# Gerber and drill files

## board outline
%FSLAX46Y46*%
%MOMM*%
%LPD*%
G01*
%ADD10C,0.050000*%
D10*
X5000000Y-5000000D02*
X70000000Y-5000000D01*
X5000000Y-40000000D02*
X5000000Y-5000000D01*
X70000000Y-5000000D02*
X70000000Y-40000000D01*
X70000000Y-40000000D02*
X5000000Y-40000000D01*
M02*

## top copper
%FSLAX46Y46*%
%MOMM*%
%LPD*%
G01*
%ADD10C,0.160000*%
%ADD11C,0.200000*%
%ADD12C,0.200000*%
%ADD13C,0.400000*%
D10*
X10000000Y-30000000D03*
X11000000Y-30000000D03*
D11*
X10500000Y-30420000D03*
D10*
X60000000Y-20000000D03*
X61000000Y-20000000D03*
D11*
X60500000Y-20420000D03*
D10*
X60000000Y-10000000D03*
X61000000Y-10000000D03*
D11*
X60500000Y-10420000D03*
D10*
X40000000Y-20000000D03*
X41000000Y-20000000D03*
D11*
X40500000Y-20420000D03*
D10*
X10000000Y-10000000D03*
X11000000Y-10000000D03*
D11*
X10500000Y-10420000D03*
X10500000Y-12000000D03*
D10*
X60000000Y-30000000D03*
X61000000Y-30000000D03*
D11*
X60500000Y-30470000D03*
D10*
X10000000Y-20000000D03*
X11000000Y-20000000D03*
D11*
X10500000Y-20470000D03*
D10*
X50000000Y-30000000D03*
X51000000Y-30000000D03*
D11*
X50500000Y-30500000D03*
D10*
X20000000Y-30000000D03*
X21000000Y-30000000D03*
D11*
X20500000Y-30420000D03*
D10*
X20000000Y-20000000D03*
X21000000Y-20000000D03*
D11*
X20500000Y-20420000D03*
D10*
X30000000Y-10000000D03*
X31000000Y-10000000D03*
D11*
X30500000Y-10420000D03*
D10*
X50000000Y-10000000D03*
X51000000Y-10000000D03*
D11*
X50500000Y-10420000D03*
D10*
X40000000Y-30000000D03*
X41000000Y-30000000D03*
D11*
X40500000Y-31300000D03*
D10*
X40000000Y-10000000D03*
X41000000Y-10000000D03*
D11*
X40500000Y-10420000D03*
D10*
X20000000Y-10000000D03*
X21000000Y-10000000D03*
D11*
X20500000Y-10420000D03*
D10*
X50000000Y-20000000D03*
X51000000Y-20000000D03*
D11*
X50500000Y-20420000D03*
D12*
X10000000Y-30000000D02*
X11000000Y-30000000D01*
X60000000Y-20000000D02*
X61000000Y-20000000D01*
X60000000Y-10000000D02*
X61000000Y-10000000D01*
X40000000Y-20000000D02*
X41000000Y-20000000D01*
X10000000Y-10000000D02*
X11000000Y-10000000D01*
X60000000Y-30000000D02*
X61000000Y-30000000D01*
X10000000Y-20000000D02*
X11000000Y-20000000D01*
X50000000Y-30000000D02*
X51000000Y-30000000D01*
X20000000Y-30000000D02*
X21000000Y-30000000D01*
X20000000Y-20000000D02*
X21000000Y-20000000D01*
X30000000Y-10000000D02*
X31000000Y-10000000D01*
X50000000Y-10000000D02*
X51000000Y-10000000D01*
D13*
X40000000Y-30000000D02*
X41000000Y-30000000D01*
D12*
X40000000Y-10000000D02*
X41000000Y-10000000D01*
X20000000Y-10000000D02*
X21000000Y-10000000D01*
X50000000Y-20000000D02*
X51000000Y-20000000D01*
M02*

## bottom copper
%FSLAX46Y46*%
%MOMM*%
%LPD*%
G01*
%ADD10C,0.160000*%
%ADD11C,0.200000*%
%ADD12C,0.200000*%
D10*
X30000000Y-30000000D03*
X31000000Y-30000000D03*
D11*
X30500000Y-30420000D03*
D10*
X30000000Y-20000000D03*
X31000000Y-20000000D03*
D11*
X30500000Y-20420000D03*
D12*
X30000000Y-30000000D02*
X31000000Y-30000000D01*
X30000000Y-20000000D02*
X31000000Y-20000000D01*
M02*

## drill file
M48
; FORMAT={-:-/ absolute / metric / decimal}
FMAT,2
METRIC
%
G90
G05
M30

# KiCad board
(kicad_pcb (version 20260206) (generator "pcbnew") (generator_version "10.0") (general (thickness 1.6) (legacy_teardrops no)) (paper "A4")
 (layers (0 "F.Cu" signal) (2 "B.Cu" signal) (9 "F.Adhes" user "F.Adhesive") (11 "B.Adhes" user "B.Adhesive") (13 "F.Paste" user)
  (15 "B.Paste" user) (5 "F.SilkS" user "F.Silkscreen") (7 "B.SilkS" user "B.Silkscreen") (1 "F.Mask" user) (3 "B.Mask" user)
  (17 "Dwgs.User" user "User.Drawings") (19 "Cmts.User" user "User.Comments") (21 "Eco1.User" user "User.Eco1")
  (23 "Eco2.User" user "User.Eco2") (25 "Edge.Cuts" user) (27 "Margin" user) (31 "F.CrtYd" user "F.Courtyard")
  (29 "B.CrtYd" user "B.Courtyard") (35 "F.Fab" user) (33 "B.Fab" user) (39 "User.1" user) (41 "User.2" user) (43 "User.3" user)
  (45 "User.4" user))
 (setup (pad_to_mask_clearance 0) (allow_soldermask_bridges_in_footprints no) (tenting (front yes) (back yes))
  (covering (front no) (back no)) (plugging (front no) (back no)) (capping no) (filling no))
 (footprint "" (layer "F.Cu") (at 10 30)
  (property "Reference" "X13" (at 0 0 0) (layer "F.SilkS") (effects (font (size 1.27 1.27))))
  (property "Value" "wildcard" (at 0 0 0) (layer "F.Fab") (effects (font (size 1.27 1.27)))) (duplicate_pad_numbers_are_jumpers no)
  (pad "1" smd circle (at 0 0) (size 0.16 0.16) (layers "F.Cu") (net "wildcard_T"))
  (pad "2" smd circle (at 1 0) (size 0.16 0.16) (layers "F.Cu") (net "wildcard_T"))
  (pad "3" smd circle (at 0.5 0.42) (size 0.2 0.2) (layers "F.Cu") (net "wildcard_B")))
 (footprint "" (layer "F.Cu") (at 60 20)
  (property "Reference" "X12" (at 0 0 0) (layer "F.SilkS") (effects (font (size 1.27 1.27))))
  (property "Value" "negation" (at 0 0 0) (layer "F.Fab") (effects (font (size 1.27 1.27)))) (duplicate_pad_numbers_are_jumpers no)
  (pad "1" smd circle (at 0 0) (size 0.16 0.16) (layers "F.Cu") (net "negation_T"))
  (pad "2" smd circle (at 1 0) (size 0.16 0.16) (layers "F.Cu") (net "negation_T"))
  (pad "3" smd circle (at 0.5 0.42) (size 0.2 0.2) (layers "F.Cu") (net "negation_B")))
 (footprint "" (layer "F.Cu") (at 60 10)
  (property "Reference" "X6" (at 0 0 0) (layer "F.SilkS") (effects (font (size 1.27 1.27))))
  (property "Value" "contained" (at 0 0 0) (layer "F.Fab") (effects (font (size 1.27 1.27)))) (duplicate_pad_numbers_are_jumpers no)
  (pad "1" smd circle (at 0 0) (size 0.16 0.16) (layers "F.Cu") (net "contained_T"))
  (pad "2" smd circle (at 1 0) (size 0.16 0.16) (layers "F.Cu") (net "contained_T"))
  (pad "3" smd circle (at 0.5 0.42) (size 0.2 0.2) (layers "F.Cu") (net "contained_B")))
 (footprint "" (layer "F.Cu") (at 40 20)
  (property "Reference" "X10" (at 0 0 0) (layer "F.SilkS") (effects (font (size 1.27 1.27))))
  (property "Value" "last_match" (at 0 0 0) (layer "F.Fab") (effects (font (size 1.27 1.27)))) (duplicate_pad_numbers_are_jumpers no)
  (pad "1" smd circle (at 0 0) (size 0.16 0.16) (layers "F.Cu") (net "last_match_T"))
  (pad "2" smd circle (at 1 0) (size 0.16 0.16) (layers "F.Cu") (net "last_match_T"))
  (pad "3" smd circle (at 0.5 0.42) (size 0.2 0.2) (layers "F.Cu") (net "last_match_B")))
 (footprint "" (layer "F.Cu") (at 10 10)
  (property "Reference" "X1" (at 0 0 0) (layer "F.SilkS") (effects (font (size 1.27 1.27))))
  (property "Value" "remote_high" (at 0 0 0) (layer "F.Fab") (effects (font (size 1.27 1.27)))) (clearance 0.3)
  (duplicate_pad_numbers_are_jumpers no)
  (pad "1" smd circle (at 0 0) (size 0.16 0.16) (layers "F.Cu") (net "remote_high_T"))
  (pad "2" smd circle (at 1 0) (size 0.16 0.16) (layers "F.Cu") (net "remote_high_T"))
  (pad "3" smd circle (at 0.5 0.42) (size 0.2 0.2) (layers "F.Cu") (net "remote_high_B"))
  (pad "4" smd circle (at 0.5 2) (size 0.2 0.2) (layers "F.Cu") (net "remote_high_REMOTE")))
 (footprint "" (layer "F.Cu") (at 60 30)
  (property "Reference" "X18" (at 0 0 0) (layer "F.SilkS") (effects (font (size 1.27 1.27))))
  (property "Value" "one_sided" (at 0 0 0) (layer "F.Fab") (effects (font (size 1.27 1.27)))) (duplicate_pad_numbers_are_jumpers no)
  (pad "1" smd circle (at 0 0) (size 0.16 0.16) (layers "F.Cu") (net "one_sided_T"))
  (pad "2" smd circle (at 1 0) (size 0.16 0.16) (layers "F.Cu") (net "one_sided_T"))
  (pad "3" smd circle (at 0.5 0.47) (size 0.2 0.2) (layers "F.Cu") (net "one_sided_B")))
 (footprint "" (layer "F.Cu") (at 10 20)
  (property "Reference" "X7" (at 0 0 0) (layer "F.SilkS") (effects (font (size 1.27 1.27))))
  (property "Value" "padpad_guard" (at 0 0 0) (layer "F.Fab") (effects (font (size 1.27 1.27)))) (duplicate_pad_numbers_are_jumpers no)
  (pad "1" smd circle (at 0 0) (size 0.16 0.16) (layers "F.Cu") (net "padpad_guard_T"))
  (pad "2" smd circle (at 1 0) (size 0.16 0.16) (layers "F.Cu") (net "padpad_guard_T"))
  (pad "3" smd circle (at 0.5 0.47) (size 0.2 0.2) (layers "F.Cu") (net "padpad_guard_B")))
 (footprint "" (layer "F.Cu") (at 50 30)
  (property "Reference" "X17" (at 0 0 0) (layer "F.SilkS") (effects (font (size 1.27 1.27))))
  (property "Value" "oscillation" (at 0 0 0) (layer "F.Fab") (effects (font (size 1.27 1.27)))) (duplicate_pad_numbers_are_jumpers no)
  (pad "1" smd circle (at 0 0) (size 0.16 0.16) (layers "F.Cu") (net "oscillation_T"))
  (pad "2" smd circle (at 1 0) (size 0.16 0.16) (layers "F.Cu") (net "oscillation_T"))
  (pad "3" smd circle (at 0.5 0.5) (size 0.2 0.2) (layers "F.Cu") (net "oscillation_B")))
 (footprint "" (layer "F.Cu") (at 20 30)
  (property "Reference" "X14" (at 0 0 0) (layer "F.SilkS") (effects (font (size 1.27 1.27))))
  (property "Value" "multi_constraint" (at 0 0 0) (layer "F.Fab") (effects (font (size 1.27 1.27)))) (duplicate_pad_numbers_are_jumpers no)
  (pad "1" smd circle (at 0 0) (size 0.16 0.16) (layers "F.Cu") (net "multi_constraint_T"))
  (pad "2" smd circle (at 1 0) (size 0.16 0.16) (layers "F.Cu") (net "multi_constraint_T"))
  (pad "3" smd circle (at 0.5 0.42) (size 0.2 0.2) (layers "F.Cu") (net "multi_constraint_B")))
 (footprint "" (layer "F.Cu") (at 30 30)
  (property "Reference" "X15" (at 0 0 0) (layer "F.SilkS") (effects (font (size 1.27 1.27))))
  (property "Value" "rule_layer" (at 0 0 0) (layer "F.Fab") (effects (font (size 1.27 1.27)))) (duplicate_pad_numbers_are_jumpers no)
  (pad "1" smd circle (at 0 0) (size 0.16 0.16) (layers "B.Cu") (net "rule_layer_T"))
  (pad "2" smd circle (at 1 0) (size 0.16 0.16) (layers "B.Cu") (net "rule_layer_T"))
  (pad "3" smd circle (at 0.5 0.42) (size 0.2 0.2) (layers "B.Cu") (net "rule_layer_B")))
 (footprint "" (layer "F.Cu") (at 20 20)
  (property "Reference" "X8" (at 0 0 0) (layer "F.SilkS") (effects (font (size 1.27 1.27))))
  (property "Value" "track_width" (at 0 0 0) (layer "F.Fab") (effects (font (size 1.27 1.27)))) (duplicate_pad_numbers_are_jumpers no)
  (pad "1" smd circle (at 0 0) (size 0.16 0.16) (layers "F.Cu") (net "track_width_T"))
  (pad "2" smd circle (at 1 0) (size 0.16 0.16) (layers "F.Cu") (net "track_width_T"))
  (pad "3" smd circle (at 0.5 0.42) (size 0.2 0.2) (layers "F.Cu") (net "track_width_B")))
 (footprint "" (layer "F.Cu") (at 30 10)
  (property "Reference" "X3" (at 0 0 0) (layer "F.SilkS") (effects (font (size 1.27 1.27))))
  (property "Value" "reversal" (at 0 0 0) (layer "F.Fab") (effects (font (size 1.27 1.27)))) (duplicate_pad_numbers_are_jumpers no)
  (pad "1" smd circle (at 0 0) (size 0.16 0.16) (layers "F.Cu") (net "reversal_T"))
  (pad "2" smd circle (at 1 0) (size 0.16 0.16) (layers "F.Cu") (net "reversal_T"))
  (pad "3" smd circle (at 0.5 0.42) (size 0.2 0.2) (layers "F.Cu") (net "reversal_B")))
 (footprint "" (layer "F.Cu") (at 50 10)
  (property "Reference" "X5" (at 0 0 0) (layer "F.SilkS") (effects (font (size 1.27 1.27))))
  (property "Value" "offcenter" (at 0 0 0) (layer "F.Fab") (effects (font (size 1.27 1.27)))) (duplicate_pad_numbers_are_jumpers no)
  (pad "1" smd circle (at 0 0) (size 0.16 0.16) (layers "F.Cu") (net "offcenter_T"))
  (pad "2" smd circle (at 1 0) (size 0.16 0.16) (layers "F.Cu") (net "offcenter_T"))
  (pad "3" smd circle (at 0.5 0.42) (size 0.2 0.2) (layers "F.Cu") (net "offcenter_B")))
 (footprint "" (layer "F.Cu") (at 40 30)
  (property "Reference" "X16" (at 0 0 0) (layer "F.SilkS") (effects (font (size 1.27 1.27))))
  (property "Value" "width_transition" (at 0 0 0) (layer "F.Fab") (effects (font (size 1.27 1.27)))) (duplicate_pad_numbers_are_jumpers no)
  (pad "1" smd circle (at 0 0) (size 0.16 0.16) (layers "F.Cu") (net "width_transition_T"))
  (pad "2" smd circle (at 1 0) (size 0.16 0.16) (layers "F.Cu") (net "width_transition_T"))
  (pad "3" smd circle (at 0.5 1.3) (size 0.2 0.2) (layers "F.Cu") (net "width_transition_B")))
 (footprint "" (layer "F.Cu") (at 30 20)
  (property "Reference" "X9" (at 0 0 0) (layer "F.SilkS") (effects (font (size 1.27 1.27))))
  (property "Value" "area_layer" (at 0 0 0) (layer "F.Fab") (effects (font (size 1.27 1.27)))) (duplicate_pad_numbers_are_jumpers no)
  (pad "1" smd circle (at 0 0) (size 0.16 0.16) (layers "B.Cu") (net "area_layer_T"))
  (pad "2" smd circle (at 1 0) (size 0.16 0.16) (layers "B.Cu") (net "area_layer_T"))
  (pad "3" smd circle (at 0.5 0.42) (size 0.2 0.2) (layers "B.Cu") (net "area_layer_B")))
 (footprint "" (layer "F.Cu") (at 40 10)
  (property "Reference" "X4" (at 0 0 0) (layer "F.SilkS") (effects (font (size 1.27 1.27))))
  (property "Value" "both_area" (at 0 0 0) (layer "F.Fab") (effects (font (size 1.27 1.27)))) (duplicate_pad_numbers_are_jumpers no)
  (pad "1" smd circle (at 0 0) (size 0.16 0.16) (layers "F.Cu") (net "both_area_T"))
  (pad "2" smd circle (at 1 0) (size 0.16 0.16) (layers "F.Cu") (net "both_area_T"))
  (pad "3" smd circle (at 0.5 0.42) (size 0.2 0.2) (layers "F.Cu") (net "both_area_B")))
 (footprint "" (layer "F.Cu") (at 20 10)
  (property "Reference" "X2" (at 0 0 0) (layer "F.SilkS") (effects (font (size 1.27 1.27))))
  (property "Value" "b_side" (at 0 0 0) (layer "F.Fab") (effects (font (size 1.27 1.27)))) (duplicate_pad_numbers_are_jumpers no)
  (pad "1" smd circle (at 0 0) (size 0.16 0.16) (layers "F.Cu") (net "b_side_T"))
  (pad "2" smd circle (at 1 0) (size 0.16 0.16) (layers "F.Cu") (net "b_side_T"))
  (pad "3" smd circle (at 0.5 0.42) (size 0.2 0.2) (layers "F.Cu") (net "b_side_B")))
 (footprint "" (layer "F.Cu") (at 50 20)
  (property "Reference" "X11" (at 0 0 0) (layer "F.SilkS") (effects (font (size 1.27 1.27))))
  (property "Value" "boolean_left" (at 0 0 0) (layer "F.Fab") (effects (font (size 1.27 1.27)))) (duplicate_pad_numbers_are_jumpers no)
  (pad "1" smd circle (at 0 0) (size 0.16 0.16) (layers "F.Cu") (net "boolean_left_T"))
  (pad "2" smd circle (at 1 0) (size 0.16 0.16) (layers "F.Cu") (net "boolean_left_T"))
  (pad "3" smd circle (at 0.5 0.42) (size 0.2 0.2) (layers "F.Cu") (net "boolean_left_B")))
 (gr_line (start 5 5) (end 70 5) (stroke (width 0.05) (type default)) (layer "Edge.Cuts"))
 (gr_line (start 5 40) (end 5 5) (stroke (width 0.05) (type default)) (layer "Edge.Cuts"))
 (gr_line (start 70 5) (end 70 40) (stroke (width 0.05) (type default)) (layer "Edge.Cuts"))
 (gr_line (start 70 40) (end 5 40) (stroke (width 0.05) (type default)) (layer "Edge.Cuts"))
 (segment (start 10 30) (end 11 30) (width 0.2) (layer "F.Cu") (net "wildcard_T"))
 (segment (start 60 20) (end 61 20) (width 0.2) (layer "F.Cu") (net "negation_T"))
 (segment (start 60 10) (end 61 10) (width 0.2) (layer "F.Cu") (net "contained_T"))
 (segment (start 40 20) (end 41 20) (width 0.2) (layer "F.Cu") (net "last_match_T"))
 (segment (start 10 10) (end 11 10) (width 0.2) (layer "F.Cu") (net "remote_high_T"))
 (segment (start 60 30) (end 61 30) (width 0.2) (layer "F.Cu") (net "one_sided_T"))
 (segment (start 10 20) (end 11 20) (width 0.2) (layer "F.Cu") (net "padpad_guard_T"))
 (segment (start 50 30) (end 51 30) (width 0.2) (layer "F.Cu") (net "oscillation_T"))
 (segment (start 20 30) (end 21 30) (width 0.2) (layer "F.Cu") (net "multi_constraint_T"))
 (segment (start 30 30) (end 31 30) (width 0.2) (layer "B.Cu") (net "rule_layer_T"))
 (segment (start 20 20) (end 21 20) (width 0.2) (layer "F.Cu") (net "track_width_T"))
 (segment (start 30 10) (end 31 10) (width 0.2) (layer "F.Cu") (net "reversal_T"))
 (segment (start 50 10) (end 51 10) (width 0.2) (layer "F.Cu") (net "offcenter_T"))
 (segment (start 40 30) (end 41 30) (width 0.4) (layer "F.Cu") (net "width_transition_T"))
 (segment (start 30 20) (end 31 20) (width 0.2) (layer "B.Cu") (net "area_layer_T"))
 (segment (start 40 10) (end 41 10) (width 0.2) (layer "F.Cu") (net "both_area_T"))
 (segment (start 20 10) (end 21 10) (width 0.2) (layer "F.Cu") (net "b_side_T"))
 (segment (start 50 20) (end 51 20) (width 0.2) (layer "F.Cu") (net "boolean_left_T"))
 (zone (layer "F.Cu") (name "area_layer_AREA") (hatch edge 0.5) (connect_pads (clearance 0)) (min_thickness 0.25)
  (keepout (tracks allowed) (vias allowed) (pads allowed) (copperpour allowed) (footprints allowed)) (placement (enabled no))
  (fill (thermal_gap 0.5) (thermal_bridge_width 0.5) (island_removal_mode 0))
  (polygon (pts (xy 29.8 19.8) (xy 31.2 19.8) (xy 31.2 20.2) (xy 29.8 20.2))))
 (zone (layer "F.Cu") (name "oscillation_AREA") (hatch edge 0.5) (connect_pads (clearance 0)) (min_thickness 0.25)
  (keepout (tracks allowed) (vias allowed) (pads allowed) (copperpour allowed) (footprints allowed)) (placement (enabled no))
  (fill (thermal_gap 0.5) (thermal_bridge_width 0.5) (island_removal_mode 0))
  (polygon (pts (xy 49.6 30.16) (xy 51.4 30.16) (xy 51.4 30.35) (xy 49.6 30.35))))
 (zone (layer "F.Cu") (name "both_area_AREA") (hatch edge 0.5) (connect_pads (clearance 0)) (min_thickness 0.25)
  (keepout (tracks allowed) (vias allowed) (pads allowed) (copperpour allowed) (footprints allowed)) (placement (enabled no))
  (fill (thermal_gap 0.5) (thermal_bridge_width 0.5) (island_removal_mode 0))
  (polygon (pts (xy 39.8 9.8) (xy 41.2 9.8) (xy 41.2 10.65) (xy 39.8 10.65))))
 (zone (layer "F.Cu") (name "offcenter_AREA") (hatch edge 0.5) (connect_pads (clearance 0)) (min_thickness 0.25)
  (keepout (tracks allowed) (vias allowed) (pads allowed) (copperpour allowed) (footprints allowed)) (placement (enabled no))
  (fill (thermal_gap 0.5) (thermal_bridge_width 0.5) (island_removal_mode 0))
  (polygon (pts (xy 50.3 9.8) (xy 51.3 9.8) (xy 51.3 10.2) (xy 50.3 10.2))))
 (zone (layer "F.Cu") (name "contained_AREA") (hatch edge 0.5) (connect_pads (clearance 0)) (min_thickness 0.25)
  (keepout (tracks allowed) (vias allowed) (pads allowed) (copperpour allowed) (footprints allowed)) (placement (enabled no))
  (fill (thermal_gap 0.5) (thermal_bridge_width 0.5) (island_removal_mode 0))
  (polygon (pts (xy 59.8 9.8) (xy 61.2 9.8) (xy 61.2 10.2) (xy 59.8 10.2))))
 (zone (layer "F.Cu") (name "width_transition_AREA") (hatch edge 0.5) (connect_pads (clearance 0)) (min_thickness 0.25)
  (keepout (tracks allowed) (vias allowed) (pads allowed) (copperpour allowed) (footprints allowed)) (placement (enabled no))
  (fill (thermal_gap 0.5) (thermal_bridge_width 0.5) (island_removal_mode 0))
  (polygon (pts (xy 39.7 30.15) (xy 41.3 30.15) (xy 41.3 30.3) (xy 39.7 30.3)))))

